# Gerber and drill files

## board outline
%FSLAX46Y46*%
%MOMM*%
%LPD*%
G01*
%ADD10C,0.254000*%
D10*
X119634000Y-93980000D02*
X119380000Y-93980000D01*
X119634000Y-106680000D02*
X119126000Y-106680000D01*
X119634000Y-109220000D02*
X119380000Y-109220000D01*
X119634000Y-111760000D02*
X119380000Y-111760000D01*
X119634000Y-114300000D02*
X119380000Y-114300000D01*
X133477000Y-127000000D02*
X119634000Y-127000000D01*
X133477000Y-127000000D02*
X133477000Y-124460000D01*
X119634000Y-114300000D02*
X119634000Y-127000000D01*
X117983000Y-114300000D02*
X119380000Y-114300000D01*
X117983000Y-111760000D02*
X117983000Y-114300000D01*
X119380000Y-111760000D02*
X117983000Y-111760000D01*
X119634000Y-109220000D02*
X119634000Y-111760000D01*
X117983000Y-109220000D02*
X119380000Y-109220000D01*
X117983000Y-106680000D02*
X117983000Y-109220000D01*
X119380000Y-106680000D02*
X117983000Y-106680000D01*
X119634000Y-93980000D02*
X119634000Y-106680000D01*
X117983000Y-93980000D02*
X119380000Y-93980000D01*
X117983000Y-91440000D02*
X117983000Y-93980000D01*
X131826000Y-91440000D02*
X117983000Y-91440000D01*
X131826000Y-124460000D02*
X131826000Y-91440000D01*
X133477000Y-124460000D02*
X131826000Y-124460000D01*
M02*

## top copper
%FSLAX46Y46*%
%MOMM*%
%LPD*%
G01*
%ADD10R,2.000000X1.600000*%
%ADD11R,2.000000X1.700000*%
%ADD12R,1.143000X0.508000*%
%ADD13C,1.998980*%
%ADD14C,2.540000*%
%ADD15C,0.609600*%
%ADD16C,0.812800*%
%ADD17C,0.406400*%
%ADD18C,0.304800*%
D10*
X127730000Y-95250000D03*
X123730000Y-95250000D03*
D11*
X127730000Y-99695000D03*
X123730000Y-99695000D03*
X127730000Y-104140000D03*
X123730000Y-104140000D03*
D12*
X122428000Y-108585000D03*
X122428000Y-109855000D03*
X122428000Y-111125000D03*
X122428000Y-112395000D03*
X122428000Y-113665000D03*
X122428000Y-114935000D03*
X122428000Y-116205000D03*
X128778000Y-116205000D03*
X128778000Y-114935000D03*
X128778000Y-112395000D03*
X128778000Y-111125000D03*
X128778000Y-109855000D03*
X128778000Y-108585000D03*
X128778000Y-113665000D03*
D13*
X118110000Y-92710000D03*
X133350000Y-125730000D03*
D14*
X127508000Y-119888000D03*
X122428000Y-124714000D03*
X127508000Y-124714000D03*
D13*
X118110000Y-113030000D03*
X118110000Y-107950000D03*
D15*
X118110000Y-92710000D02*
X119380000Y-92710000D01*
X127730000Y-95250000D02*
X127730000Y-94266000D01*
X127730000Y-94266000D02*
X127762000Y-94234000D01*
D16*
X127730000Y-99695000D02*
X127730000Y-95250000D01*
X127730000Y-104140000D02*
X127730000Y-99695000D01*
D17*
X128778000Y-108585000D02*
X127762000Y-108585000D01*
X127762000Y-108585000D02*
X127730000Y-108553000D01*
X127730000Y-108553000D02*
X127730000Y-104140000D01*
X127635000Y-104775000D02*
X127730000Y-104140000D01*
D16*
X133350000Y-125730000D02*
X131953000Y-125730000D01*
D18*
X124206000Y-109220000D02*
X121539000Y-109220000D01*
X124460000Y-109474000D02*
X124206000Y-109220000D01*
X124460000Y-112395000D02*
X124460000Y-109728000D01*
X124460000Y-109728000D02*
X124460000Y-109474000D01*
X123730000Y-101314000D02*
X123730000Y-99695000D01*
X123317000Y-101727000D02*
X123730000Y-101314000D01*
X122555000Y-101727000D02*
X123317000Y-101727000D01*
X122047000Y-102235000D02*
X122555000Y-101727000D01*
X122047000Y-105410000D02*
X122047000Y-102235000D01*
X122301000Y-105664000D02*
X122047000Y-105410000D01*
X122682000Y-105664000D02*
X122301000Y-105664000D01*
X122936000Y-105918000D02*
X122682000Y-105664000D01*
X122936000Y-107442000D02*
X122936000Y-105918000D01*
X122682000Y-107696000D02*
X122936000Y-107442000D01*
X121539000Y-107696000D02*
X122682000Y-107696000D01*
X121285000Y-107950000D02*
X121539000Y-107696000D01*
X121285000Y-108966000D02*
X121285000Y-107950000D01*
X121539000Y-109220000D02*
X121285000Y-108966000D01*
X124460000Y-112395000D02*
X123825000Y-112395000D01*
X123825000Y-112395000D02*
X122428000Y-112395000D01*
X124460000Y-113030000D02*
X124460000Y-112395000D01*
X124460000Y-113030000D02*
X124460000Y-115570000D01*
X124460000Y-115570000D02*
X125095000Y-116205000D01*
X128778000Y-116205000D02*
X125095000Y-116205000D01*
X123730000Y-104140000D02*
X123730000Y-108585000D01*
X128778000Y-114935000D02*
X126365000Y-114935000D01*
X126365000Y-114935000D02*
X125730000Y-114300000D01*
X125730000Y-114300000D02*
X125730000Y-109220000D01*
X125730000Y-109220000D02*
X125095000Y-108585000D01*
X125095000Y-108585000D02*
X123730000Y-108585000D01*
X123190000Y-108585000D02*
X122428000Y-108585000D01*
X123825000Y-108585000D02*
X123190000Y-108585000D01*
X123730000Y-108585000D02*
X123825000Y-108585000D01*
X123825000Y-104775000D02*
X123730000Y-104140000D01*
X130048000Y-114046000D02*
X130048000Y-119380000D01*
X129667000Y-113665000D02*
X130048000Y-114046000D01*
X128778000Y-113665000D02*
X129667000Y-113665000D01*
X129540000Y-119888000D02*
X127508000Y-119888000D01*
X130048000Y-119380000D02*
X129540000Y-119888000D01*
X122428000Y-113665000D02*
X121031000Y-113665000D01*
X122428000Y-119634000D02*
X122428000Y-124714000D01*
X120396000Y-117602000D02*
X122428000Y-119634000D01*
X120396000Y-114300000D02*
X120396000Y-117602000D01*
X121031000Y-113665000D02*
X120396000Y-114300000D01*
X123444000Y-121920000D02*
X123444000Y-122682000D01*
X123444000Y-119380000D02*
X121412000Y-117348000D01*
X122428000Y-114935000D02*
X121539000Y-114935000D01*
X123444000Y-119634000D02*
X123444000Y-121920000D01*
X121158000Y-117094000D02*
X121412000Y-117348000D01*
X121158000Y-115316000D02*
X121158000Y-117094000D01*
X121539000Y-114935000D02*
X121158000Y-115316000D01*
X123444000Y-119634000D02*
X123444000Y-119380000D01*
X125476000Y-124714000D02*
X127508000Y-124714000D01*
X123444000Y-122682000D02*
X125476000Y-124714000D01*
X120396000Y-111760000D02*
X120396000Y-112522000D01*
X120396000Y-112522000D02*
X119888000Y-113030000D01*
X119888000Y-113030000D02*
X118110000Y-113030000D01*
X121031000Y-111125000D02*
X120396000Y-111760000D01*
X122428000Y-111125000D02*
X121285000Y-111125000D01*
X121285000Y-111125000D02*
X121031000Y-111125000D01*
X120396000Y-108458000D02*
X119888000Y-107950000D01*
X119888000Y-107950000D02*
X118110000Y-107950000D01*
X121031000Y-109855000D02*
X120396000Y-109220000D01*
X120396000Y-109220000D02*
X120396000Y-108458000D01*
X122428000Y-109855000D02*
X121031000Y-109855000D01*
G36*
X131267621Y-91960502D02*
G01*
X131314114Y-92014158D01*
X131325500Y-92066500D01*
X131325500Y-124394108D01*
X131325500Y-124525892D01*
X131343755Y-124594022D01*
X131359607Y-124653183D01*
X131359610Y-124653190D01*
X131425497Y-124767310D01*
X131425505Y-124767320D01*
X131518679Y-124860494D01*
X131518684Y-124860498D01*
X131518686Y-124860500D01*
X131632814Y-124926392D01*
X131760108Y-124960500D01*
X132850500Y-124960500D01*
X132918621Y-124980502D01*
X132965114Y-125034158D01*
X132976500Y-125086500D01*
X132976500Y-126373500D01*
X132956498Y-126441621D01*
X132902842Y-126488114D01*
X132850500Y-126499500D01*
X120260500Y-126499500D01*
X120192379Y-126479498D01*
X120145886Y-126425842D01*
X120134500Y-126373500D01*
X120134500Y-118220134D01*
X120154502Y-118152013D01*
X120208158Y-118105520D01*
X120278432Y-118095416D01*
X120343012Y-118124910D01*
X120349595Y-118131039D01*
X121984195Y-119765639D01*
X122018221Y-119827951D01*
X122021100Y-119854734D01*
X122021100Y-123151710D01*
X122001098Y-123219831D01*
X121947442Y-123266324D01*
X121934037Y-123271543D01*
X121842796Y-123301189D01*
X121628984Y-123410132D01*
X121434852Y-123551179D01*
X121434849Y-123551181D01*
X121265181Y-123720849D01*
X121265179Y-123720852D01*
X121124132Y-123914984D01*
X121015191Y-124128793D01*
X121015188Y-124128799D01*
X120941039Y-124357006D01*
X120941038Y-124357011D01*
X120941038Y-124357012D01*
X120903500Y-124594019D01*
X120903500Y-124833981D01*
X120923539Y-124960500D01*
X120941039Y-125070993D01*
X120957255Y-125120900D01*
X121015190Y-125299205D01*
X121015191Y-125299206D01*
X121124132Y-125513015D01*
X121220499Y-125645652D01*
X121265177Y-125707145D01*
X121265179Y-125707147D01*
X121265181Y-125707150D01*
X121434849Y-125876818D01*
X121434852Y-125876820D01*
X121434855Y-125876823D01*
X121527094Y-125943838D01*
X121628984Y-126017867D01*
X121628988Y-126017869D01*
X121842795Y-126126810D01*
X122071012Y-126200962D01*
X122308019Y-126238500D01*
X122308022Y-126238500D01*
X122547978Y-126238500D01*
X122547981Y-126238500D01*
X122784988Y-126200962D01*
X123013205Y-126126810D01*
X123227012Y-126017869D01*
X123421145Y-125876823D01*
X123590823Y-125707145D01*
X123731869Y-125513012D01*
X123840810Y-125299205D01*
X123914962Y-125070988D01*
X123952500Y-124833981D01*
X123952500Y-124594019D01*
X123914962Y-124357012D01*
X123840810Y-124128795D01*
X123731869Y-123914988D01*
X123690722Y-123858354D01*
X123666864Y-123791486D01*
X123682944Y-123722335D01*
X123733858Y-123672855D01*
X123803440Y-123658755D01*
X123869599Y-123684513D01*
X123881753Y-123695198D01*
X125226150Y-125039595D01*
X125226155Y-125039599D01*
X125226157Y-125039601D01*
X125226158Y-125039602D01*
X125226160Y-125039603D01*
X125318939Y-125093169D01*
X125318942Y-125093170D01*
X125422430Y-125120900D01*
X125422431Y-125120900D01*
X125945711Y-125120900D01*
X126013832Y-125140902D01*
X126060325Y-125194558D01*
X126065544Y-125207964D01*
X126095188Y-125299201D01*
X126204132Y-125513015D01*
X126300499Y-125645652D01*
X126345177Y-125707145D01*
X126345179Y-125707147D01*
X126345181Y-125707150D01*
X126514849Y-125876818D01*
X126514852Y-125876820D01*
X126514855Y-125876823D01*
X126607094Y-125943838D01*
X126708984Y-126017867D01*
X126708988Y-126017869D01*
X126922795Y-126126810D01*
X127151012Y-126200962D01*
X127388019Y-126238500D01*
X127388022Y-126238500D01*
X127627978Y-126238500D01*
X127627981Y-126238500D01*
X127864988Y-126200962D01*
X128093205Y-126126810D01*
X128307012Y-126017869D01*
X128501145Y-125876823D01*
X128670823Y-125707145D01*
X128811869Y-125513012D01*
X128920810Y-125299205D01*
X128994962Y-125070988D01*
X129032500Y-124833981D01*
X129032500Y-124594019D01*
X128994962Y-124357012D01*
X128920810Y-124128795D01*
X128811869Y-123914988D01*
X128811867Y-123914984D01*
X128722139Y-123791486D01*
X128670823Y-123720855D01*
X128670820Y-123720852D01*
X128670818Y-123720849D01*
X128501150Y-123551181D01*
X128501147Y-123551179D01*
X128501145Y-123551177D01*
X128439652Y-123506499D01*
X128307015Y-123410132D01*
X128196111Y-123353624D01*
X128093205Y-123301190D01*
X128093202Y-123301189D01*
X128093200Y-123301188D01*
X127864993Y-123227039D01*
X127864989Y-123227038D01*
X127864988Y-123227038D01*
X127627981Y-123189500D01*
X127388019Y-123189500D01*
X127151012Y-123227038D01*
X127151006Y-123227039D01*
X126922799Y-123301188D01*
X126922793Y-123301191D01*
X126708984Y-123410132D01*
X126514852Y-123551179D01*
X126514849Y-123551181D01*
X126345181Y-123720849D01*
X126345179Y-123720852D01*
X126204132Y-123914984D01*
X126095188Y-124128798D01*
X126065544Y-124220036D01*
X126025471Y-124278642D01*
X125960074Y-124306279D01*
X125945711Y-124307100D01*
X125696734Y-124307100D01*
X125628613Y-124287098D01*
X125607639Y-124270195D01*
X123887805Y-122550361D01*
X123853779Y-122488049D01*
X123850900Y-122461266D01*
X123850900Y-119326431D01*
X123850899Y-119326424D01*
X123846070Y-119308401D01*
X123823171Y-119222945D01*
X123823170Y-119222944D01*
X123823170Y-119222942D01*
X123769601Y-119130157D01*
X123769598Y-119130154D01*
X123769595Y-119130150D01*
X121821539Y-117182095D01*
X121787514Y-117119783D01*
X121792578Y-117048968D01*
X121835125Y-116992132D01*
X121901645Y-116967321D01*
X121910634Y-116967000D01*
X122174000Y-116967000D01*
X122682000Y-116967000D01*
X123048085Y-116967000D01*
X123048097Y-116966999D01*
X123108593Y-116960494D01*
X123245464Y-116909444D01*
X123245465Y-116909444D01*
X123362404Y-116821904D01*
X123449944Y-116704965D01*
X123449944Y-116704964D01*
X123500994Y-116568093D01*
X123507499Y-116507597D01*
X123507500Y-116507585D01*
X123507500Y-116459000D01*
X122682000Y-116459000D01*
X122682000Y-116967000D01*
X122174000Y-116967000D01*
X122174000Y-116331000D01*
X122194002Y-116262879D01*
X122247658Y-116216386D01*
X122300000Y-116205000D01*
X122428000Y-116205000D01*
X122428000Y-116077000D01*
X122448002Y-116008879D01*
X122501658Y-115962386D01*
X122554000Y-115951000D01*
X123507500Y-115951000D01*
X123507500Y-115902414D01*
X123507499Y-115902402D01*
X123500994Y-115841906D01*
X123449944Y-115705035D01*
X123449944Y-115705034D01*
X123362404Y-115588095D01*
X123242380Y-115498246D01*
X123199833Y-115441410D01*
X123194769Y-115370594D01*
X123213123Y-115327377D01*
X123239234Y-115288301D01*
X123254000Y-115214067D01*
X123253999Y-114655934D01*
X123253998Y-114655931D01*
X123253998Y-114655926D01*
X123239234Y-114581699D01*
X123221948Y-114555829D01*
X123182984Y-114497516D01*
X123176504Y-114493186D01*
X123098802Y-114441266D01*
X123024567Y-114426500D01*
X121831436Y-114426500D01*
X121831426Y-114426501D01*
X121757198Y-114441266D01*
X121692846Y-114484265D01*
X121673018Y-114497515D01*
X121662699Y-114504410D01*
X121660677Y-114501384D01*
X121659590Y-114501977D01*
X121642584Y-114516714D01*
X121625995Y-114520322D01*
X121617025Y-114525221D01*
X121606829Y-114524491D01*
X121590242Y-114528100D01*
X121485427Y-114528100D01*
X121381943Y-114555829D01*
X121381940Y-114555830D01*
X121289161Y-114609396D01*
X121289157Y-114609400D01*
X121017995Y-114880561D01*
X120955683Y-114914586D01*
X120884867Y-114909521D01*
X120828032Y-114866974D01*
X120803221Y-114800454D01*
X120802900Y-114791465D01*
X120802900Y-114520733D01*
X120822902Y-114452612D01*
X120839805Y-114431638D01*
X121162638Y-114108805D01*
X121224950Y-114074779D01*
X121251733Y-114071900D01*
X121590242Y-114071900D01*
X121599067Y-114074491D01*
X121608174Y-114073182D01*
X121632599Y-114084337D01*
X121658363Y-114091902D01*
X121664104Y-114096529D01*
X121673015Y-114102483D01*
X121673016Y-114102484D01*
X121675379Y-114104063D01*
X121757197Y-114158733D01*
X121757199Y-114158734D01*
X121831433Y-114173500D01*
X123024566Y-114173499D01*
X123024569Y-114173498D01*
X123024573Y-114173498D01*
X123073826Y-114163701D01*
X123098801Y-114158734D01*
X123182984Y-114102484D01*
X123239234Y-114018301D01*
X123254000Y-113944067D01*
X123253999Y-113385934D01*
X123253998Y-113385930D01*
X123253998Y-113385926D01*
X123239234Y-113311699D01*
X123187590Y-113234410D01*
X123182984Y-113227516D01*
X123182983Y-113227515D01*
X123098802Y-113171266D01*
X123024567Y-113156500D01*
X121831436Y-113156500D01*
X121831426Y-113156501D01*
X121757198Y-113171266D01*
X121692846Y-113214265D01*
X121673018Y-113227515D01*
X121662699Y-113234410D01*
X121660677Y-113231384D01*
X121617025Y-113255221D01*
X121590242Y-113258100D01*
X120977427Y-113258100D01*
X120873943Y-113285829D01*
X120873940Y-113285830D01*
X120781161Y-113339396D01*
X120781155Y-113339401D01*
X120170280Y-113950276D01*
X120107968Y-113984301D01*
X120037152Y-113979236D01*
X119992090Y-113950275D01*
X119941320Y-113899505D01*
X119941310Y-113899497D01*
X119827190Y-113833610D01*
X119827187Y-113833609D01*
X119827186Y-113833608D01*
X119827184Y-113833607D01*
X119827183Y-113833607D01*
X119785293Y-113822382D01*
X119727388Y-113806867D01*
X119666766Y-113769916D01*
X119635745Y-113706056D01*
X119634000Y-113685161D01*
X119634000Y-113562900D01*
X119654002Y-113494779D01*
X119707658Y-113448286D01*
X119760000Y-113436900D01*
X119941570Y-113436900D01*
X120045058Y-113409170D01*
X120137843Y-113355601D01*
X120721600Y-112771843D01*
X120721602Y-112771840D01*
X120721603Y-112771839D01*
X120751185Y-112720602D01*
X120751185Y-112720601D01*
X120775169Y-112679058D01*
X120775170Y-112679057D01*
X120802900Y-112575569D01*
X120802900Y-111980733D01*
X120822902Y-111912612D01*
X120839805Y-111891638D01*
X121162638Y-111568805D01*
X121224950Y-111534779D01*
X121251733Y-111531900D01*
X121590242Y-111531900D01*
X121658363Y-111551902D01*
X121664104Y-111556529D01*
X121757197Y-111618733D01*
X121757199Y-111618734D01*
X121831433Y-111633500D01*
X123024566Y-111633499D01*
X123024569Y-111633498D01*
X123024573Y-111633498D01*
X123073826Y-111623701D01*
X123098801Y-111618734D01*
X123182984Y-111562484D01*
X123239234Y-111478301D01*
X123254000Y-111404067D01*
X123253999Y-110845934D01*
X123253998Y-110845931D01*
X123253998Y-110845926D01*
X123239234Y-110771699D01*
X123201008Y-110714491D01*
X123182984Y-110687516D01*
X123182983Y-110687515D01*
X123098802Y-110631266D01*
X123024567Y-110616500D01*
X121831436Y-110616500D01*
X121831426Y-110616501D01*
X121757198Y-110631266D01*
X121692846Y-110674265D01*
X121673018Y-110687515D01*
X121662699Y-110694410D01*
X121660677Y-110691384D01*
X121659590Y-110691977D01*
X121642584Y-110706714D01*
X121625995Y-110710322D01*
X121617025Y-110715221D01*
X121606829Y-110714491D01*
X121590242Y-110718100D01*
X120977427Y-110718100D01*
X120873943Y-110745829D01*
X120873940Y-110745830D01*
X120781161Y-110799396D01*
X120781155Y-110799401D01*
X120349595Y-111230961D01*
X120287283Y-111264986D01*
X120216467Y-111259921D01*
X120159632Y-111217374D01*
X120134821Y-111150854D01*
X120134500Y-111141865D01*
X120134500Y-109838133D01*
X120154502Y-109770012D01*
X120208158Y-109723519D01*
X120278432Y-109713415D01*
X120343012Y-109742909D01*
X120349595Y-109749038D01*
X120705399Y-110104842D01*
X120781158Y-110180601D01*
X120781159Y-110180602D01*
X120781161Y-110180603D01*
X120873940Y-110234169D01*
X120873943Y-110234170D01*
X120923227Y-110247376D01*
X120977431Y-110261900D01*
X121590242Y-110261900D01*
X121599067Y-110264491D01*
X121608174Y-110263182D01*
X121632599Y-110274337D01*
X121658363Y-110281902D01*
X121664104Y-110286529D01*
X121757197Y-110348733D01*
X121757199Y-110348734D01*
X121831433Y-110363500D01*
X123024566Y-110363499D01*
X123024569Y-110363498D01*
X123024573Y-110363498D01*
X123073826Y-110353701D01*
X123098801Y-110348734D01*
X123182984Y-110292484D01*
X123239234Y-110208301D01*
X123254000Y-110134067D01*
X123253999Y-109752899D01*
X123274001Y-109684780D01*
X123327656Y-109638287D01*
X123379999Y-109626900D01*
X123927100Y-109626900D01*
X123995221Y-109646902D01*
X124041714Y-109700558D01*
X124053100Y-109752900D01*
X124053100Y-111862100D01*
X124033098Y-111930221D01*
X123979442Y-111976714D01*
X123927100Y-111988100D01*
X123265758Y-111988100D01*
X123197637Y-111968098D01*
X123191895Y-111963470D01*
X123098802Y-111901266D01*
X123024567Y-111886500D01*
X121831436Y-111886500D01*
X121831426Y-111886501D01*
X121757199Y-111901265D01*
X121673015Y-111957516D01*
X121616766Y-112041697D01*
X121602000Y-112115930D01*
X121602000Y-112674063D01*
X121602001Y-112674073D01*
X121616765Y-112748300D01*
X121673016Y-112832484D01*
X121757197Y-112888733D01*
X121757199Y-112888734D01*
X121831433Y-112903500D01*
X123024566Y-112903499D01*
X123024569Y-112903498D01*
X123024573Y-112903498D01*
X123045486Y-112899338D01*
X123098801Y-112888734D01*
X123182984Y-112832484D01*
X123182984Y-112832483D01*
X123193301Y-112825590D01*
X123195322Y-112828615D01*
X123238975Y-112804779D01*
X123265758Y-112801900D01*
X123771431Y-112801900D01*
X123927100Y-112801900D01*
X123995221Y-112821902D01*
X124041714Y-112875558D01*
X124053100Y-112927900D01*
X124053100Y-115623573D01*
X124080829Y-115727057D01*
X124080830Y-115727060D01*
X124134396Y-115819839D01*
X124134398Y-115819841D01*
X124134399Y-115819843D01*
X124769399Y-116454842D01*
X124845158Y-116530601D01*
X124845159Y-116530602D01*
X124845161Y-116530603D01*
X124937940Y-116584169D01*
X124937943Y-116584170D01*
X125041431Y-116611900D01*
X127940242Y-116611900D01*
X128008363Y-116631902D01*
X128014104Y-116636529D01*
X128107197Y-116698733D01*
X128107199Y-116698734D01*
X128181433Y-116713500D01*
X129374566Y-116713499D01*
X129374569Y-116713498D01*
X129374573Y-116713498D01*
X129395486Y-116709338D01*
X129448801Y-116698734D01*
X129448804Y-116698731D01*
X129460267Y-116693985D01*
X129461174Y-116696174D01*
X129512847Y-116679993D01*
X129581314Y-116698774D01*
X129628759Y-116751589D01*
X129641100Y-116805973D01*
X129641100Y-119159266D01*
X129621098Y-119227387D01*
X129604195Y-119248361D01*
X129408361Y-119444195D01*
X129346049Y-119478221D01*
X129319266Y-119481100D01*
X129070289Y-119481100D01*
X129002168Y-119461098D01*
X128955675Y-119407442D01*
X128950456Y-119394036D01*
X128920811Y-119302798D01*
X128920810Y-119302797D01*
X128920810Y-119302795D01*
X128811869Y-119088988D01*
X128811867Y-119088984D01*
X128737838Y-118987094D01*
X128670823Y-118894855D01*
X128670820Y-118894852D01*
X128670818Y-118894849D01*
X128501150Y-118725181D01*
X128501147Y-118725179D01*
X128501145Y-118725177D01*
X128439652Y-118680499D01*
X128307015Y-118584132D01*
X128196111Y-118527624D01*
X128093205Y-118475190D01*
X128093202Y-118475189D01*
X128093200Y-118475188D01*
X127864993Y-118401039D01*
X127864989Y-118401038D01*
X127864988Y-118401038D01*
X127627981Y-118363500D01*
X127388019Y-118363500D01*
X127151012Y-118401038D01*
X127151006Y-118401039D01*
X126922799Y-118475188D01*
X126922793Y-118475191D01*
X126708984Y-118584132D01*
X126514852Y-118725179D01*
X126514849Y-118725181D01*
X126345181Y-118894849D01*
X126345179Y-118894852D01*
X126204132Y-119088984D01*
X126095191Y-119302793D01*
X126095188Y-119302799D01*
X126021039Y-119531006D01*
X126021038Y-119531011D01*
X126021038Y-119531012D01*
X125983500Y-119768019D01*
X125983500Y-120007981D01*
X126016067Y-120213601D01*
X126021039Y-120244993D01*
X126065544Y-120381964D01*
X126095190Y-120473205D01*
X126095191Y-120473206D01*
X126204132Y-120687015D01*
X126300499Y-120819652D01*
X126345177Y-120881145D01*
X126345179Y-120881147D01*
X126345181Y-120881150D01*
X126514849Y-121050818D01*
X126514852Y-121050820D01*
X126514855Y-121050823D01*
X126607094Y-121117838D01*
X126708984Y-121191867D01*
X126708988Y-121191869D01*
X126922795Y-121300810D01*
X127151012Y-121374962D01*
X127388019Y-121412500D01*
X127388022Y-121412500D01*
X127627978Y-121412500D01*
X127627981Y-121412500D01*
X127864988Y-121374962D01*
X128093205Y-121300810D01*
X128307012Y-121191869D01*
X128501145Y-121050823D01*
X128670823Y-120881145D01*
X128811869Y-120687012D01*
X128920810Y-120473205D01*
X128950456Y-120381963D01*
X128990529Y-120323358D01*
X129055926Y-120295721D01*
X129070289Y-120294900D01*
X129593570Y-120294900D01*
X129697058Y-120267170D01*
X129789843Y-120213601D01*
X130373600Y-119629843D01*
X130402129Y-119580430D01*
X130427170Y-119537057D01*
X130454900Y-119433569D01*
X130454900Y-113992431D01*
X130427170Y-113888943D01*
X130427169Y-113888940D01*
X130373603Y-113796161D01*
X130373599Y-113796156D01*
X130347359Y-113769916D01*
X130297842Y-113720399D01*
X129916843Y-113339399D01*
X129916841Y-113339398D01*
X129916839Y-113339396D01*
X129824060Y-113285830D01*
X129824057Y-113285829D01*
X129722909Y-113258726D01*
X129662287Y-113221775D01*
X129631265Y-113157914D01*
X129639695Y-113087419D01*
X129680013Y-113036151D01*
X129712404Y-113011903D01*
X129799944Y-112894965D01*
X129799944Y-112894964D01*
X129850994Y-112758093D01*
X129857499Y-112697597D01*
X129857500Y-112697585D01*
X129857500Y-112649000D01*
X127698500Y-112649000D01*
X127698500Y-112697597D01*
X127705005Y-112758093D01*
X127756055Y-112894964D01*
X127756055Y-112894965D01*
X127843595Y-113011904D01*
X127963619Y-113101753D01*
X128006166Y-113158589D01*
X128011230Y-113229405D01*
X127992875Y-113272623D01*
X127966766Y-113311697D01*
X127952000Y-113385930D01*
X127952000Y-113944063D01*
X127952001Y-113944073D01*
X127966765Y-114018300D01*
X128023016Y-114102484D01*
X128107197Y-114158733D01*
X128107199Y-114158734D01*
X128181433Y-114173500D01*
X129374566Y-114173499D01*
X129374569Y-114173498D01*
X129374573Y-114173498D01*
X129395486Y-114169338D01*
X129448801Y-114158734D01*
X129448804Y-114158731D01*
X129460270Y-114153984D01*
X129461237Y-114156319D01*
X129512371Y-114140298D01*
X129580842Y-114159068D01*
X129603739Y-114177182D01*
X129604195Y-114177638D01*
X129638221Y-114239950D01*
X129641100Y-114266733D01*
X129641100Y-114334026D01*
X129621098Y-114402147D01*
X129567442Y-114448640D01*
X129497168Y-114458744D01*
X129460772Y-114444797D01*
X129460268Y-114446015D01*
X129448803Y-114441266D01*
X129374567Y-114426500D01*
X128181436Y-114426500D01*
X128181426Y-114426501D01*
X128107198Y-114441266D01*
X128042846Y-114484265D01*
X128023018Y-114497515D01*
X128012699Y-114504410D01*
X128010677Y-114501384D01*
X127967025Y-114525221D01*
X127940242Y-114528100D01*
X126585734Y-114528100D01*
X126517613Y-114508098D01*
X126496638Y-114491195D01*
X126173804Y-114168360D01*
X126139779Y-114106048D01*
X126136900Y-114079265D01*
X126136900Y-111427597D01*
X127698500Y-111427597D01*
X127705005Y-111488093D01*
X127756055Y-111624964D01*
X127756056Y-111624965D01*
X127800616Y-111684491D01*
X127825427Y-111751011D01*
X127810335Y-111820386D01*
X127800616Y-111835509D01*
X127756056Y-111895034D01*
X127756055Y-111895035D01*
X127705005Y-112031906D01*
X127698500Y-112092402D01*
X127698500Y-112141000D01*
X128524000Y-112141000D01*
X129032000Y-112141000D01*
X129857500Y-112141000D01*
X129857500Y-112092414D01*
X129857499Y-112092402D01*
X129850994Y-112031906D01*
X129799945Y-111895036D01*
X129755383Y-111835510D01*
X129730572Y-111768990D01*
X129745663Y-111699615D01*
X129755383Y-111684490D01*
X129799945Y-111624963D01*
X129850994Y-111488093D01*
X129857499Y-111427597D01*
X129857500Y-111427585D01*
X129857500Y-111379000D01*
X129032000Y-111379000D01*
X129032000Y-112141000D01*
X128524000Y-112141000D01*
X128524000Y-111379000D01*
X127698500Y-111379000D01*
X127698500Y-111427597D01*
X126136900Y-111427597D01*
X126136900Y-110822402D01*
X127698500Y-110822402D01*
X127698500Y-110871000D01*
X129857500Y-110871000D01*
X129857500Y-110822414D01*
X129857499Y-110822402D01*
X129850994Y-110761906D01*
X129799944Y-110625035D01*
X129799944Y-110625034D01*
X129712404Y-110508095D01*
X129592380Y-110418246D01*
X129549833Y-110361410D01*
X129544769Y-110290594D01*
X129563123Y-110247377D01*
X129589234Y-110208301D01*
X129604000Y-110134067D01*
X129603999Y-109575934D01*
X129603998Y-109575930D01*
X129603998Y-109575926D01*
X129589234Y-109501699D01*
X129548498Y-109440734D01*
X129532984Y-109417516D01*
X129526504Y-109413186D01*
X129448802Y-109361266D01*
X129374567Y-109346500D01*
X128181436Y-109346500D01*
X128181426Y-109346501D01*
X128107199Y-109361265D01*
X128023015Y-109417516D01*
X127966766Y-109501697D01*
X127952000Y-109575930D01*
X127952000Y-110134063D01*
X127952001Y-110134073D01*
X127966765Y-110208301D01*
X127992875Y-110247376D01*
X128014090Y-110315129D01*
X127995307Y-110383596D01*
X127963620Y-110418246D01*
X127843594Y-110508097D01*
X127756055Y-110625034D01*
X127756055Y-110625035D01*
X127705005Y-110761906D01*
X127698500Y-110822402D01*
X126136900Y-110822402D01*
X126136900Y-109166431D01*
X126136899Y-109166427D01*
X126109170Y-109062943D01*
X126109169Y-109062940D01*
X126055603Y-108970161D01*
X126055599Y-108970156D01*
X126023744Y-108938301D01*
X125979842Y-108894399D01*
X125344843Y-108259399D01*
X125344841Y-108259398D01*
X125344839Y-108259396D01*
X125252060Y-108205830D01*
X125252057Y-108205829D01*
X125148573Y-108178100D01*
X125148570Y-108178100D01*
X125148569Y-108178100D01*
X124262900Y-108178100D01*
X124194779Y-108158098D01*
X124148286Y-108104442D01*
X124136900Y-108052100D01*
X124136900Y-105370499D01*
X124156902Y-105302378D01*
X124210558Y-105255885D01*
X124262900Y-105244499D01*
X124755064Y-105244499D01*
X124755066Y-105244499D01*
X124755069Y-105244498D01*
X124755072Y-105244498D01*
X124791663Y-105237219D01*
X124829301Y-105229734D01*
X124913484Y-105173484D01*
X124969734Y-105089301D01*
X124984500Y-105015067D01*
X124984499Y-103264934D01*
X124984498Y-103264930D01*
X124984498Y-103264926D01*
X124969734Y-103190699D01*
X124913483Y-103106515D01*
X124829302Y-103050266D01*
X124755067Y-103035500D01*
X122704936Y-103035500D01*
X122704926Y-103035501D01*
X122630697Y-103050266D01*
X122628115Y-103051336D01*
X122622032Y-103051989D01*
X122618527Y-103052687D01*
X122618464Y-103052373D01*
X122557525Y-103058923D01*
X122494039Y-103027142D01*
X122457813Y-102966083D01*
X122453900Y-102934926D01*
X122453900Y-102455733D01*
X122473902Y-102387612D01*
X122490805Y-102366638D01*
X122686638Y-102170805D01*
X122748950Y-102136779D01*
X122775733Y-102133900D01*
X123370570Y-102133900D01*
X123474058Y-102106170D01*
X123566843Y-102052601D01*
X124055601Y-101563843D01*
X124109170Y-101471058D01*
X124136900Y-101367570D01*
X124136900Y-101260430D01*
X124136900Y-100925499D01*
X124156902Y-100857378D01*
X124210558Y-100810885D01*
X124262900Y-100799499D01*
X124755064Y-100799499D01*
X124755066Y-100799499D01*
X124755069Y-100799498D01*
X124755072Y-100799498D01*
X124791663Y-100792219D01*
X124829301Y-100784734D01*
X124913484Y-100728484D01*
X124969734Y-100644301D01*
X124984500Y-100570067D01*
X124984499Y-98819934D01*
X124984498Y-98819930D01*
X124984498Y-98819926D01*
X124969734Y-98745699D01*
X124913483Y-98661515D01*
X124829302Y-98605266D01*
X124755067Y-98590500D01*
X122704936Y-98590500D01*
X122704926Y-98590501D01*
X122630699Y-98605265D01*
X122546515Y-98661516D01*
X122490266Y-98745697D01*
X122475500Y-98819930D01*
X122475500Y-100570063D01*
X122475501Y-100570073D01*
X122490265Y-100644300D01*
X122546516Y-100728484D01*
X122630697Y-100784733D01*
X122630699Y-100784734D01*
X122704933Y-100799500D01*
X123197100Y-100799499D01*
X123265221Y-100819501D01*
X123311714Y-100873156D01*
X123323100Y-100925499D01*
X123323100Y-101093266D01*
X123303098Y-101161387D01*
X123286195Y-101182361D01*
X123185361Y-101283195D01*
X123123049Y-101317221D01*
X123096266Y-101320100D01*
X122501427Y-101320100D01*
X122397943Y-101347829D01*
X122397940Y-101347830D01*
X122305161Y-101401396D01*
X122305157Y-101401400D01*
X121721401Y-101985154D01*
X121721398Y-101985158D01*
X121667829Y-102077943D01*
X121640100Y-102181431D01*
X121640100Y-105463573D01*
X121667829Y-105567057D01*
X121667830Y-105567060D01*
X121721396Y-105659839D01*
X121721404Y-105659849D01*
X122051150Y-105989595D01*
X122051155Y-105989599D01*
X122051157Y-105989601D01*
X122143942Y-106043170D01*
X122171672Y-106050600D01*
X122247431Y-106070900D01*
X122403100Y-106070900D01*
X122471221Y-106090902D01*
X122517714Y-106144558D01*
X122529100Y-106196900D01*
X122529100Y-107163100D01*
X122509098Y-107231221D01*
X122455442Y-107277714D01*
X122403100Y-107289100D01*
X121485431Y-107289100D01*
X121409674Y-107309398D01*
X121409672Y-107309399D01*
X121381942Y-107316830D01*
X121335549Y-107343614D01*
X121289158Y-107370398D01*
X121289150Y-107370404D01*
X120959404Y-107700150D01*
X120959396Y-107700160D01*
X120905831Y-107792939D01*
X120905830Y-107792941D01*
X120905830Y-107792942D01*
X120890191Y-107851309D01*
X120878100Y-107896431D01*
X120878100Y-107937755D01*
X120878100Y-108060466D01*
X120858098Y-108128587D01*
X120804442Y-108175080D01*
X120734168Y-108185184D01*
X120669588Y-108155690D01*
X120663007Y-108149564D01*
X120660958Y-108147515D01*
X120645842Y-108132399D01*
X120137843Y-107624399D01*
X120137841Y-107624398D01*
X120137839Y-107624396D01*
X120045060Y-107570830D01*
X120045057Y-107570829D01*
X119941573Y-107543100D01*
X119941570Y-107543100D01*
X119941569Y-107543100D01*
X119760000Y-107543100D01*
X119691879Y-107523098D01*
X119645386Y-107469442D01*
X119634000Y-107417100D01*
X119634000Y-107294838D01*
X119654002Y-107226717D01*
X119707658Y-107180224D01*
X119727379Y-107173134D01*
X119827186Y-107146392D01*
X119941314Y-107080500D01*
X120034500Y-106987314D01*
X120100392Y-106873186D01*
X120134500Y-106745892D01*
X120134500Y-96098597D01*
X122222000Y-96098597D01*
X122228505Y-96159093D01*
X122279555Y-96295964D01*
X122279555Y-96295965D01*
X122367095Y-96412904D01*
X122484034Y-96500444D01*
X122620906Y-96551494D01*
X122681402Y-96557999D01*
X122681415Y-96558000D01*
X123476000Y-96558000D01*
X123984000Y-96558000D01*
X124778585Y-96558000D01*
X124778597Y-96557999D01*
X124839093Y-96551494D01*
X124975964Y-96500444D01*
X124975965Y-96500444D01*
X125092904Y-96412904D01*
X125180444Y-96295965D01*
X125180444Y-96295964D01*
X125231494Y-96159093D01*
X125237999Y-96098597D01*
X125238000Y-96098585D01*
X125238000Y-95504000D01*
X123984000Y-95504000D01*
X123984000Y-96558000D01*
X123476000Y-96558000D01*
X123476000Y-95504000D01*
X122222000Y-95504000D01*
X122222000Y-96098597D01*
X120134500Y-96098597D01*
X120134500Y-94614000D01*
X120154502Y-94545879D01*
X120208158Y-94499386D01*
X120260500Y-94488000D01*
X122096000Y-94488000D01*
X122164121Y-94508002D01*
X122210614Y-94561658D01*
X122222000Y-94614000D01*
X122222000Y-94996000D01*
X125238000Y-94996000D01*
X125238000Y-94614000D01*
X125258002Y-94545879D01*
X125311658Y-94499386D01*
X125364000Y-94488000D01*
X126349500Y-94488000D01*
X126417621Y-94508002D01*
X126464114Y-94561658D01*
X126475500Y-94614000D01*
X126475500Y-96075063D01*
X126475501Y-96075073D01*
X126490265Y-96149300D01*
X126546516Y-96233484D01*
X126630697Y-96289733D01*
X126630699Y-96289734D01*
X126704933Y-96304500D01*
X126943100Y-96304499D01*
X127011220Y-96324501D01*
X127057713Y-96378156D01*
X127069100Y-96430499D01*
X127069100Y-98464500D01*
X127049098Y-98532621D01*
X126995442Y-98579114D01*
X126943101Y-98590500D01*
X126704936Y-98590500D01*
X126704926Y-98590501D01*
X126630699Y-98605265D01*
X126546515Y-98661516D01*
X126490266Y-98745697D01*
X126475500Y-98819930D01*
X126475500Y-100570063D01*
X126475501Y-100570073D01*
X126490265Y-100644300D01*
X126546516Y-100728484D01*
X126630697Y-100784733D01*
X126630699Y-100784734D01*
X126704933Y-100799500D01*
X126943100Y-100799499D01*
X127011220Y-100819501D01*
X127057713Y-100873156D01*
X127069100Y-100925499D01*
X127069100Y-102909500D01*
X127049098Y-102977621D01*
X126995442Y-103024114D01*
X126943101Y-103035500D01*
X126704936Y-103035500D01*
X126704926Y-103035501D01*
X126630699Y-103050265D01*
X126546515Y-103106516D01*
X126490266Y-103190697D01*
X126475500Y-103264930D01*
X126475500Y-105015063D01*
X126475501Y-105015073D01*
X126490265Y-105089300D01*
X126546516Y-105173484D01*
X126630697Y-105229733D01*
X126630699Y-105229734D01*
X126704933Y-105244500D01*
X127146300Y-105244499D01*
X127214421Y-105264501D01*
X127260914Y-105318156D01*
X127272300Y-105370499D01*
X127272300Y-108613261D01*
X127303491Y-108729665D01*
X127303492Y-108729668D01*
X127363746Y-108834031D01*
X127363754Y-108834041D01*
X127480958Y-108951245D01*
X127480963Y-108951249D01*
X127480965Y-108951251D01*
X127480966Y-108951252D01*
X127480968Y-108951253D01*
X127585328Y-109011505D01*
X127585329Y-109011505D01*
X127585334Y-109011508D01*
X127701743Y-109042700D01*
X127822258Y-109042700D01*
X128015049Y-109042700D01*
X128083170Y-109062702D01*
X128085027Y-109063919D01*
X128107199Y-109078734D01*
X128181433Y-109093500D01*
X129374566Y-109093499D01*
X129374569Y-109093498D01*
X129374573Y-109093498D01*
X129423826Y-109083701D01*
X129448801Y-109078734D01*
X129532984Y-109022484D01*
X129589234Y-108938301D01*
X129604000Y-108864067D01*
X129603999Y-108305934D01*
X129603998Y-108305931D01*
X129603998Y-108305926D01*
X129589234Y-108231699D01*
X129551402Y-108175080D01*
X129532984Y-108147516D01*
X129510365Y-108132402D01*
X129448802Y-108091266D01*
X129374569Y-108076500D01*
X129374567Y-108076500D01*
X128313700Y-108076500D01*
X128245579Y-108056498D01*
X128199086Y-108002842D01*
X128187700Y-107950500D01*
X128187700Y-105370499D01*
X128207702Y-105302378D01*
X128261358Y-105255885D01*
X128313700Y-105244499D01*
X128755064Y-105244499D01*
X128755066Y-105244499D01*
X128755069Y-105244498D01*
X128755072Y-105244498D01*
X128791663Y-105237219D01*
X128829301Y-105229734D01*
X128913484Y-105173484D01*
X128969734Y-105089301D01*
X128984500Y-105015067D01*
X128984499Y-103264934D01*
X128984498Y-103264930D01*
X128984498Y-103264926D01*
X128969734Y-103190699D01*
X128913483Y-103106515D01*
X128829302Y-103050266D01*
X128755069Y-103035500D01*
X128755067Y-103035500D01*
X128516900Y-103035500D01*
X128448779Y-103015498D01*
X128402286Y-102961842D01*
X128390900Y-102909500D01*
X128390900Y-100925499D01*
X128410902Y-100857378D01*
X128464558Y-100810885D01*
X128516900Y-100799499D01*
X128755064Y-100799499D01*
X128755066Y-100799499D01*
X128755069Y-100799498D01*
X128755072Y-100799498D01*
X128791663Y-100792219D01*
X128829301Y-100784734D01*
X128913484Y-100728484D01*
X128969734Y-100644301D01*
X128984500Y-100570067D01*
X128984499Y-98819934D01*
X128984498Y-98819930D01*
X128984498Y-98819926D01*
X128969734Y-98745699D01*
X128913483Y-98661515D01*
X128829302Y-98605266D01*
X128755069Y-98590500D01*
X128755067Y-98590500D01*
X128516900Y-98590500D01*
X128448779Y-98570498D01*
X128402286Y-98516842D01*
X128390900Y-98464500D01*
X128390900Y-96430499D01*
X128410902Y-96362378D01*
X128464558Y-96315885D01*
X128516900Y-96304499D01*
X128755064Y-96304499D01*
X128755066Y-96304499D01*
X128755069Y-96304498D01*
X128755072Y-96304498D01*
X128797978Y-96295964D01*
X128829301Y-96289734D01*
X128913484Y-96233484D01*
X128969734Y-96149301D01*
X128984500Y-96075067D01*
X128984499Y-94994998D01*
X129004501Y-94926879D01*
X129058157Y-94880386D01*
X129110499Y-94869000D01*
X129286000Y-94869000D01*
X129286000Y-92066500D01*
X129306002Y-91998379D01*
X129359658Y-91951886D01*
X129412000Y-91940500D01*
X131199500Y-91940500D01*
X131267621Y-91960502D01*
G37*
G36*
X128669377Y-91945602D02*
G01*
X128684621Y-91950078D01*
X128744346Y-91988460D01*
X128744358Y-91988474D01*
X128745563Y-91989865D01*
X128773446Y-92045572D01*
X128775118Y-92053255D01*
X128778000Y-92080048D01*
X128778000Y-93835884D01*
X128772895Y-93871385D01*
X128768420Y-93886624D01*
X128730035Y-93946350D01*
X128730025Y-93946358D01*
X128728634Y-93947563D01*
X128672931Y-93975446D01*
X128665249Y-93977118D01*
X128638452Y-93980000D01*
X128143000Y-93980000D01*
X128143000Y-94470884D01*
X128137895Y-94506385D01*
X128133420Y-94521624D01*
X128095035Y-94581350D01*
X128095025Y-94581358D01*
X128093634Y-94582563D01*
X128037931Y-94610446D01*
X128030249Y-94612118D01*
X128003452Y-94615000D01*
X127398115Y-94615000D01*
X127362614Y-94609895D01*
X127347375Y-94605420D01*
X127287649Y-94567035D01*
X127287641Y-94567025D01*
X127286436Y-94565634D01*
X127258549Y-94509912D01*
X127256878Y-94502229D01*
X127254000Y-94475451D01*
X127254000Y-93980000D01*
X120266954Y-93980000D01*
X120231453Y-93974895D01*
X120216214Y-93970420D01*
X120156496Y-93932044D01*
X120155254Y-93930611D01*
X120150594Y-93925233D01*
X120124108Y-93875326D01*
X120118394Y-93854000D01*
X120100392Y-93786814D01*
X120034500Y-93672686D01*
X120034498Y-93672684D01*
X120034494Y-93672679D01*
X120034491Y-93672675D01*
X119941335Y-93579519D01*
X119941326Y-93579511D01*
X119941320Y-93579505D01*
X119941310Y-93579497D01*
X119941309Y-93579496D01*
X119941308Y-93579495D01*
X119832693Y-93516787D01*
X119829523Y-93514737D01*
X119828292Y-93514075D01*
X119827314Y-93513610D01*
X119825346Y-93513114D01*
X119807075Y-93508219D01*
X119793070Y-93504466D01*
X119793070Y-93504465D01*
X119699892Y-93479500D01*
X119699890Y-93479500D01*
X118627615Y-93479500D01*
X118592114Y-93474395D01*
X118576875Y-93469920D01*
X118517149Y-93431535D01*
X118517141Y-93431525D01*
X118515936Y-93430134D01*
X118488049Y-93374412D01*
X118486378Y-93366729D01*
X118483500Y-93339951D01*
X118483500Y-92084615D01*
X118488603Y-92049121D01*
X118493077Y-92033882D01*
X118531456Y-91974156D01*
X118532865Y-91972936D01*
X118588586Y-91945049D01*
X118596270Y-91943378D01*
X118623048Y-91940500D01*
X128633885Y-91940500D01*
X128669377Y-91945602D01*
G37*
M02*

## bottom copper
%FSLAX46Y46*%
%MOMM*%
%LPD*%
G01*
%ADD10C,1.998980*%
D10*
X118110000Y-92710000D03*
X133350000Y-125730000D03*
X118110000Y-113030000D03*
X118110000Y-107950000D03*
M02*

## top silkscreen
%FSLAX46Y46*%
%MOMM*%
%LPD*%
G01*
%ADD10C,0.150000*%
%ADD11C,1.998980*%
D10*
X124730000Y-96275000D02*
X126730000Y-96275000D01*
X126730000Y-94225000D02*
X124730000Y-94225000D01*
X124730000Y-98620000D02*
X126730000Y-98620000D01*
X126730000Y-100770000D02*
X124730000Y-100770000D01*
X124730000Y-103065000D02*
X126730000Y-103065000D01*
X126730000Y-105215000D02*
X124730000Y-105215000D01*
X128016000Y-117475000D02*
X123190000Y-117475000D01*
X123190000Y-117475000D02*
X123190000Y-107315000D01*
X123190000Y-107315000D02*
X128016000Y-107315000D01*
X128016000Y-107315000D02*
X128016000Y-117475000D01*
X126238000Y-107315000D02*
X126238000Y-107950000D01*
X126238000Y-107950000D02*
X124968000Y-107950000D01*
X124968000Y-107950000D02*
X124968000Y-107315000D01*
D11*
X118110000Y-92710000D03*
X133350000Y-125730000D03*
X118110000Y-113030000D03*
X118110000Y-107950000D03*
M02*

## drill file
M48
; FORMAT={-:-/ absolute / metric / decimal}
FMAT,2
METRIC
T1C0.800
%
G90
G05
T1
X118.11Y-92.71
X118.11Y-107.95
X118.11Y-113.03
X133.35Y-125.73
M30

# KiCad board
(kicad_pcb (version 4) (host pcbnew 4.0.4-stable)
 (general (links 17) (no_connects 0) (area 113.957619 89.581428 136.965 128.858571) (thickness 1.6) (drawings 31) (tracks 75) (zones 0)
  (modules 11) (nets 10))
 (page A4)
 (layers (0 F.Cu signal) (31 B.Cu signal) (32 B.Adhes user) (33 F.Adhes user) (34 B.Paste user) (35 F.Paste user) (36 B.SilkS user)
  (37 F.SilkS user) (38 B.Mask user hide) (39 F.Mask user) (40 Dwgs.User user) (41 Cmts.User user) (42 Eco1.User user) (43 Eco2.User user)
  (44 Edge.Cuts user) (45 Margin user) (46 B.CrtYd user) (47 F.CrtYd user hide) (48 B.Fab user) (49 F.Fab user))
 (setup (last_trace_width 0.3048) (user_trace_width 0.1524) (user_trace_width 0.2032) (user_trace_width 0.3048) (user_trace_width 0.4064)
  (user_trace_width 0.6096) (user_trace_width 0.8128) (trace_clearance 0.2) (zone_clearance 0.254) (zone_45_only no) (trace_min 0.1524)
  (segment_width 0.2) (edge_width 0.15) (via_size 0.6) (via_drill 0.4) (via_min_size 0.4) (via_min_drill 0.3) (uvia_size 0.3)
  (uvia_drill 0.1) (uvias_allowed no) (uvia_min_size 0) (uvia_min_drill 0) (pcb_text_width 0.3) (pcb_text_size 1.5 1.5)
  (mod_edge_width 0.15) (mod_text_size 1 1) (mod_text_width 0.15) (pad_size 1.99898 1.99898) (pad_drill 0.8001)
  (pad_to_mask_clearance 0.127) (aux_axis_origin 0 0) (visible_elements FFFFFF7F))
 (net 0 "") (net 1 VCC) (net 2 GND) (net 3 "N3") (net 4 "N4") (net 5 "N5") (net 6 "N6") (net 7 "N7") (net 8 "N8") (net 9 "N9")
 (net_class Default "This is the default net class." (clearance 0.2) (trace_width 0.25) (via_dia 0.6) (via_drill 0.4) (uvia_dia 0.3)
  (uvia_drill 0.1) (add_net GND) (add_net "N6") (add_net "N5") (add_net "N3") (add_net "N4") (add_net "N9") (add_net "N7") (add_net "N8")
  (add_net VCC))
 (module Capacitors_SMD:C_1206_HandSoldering (layer F.Cu) (at 125.73 95.25 180)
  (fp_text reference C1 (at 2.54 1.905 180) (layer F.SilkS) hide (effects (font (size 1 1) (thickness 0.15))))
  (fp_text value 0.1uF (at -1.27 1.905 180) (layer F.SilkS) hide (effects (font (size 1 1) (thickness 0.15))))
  (fp_line (start 1 -1.025) (end -1 -1.025) (layer F.SilkS) (width 0.15))
  (fp_line (start -1 1.025) (end 1 1.025) (layer F.SilkS) (width 0.15))
  (pad 1 smd rect (at -2 0 180) (size 2 1.6) (layers F.Cu F.Paste F.Mask) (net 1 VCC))
  (pad 2 smd rect (at 2 0 180) (size 2 1.6) (layers F.Cu F.Paste F.Mask) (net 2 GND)))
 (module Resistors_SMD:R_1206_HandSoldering (layer F.Cu) (at 125.73 99.695 180)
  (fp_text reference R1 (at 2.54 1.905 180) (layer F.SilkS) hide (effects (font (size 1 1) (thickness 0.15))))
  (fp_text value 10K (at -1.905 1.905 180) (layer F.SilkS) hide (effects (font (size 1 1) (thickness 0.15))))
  (fp_line (start 1 1.075) (end -1 1.075) (layer F.SilkS) (width 0.15))
  (fp_line (start -1 -1.075) (end 1 -1.075) (layer F.SilkS) (width 0.15))
  (pad 1 smd rect (at -2 0 180) (size 2 1.7) (layers F.Cu F.Paste F.Mask) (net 1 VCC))
  (pad 2 smd rect (at 2 0 180) (size 2 1.7) (layers F.Cu F.Paste F.Mask) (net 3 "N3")))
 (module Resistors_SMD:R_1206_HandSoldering (layer F.Cu) (at 125.73 104.14 180)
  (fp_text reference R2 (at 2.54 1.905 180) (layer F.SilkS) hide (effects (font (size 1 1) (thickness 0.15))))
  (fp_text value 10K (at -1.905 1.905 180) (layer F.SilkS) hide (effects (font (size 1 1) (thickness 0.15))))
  (fp_line (start 1 1.075) (end -1 1.075) (layer F.SilkS) (width 0.15))
  (fp_line (start -1 -1.075) (end 1 -1.075) (layer F.SilkS) (width 0.15))
  (pad 1 smd rect (at -2 0 180) (size 2 1.7) (layers F.Cu F.Paste F.Mask) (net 1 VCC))
  (pad 2 smd rect (at 2 0 180) (size 2 1.7) (layers F.Cu F.Paste F.Mask) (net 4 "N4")))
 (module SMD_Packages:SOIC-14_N (layer F.Cu) (at 125.73 112.395 270)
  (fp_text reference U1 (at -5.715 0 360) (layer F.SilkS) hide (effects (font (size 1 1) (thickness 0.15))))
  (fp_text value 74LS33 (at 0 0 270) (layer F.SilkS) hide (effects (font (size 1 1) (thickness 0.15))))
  (fp_line (start 5.08 -2.286) (end 5.08 2.54) (layer F.SilkS) (width 0.15))
  (fp_line (start 5.08 2.54) (end -5.08 2.54) (layer F.SilkS) (width 0.15))
  (fp_line (start -5.08 2.54) (end -5.08 -2.286) (layer F.SilkS) (width 0.15))
  (fp_line (start -5.08 -2.286) (end 5.08 -2.286) (layer F.SilkS) (width 0.15))
  (fp_line (start -5.08 -0.508) (end -4.445 -0.508) (layer F.SilkS) (width 0.15))
  (fp_line (start -4.445 -0.508) (end -4.445 0.762) (layer F.SilkS) (width 0.15))
  (fp_line (start -4.445 0.762) (end -5.08 0.762) (layer F.SilkS) (width 0.15))
  (pad 1 smd rect (at -3.81 3.302 270) (size 0.508 1.143) (layers F.Cu F.Paste F.Mask) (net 4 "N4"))
  (pad 2 smd rect (at -2.54 3.302 270) (size 0.508 1.143) (layers F.Cu F.Paste F.Mask) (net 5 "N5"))
  (pad 3 smd rect (at -1.27 3.302 270) (size 0.508 1.143) (layers F.Cu F.Paste F.Mask) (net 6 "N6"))
  (pad 4 smd rect (at 0 3.302 270) (size 0.508 1.143) (layers F.Cu F.Paste F.Mask) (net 3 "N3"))
  (pad 5 smd rect (at 1.27 3.302 270) (size 0.508 1.143) (layers F.Cu F.Paste F.Mask) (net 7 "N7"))
  (pad 6 smd rect (at 2.54 3.302 270) (size 0.508 1.143) (layers F.Cu F.Paste F.Mask) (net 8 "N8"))
  (pad 7 smd rect (at 3.81 3.302 270) (size 0.508 1.143) (layers F.Cu F.Paste F.Mask) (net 2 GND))
  (pad 8 smd rect (at 3.81 -3.048 270) (size 0.508 1.143) (layers F.Cu F.Paste F.Mask) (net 3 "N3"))
  (pad 9 smd rect (at 2.54 -3.048 270) (size 0.508 1.143) (layers F.Cu F.Paste F.Mask) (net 4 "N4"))
  (pad 11 smd rect (at 0 -3.048 270) (size 0.508 1.143) (layers F.Cu F.Paste F.Mask) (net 2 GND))
  (pad 12 smd rect (at -1.27 -3.048 270) (size 0.508 1.143) (layers F.Cu F.Paste F.Mask) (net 2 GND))
  (pad 13 smd rect (at -2.54 -3.048 270) (size 0.508 1.143) (layers F.Cu F.Paste F.Mask))
  (pad 14 smd rect (at -3.81 -3.048 270) (size 0.508 1.143) (layers F.Cu F.Paste F.Mask) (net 1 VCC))
  (pad 10 smd rect (at 1.27 -3.048 270) (size 0.508 1.143) (layers F.Cu F.Paste F.Mask) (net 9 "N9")))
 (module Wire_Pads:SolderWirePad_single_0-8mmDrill (layer F.Cu) (at 118.11 92.71 90)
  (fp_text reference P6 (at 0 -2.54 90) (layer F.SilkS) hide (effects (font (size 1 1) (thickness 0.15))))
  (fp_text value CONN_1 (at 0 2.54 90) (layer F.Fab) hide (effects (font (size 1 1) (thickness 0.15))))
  (pad 1 thru_hole circle (at 0 0 90) (size 1.99898 1.99898) (drill 0.8001) (layers *.Cu *.Mask F.SilkS) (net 1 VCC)))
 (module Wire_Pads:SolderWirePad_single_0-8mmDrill (layer F.Cu) (at 133.35 125.73 270)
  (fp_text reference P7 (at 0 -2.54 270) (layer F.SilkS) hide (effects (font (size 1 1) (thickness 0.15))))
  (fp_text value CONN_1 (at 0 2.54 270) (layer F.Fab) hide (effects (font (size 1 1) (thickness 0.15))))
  (pad 1 thru_hole circle (at 0 0 270) (size 1.99898 1.99898) (drill 0.8001) (layers *.Cu *.Mask F.SilkS) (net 2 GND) (zone_connect 2)))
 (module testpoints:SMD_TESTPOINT (layer F.Cu) (at 127.508 119.888)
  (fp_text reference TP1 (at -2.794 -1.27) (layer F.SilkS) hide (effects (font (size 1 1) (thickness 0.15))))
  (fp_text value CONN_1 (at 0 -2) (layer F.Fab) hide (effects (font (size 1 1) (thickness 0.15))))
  (pad 1 smd circle (at 0 0) (size 2.54 2.54) (layers F.Cu F.Paste F.Mask) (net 9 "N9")))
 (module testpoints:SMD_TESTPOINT (layer F.Cu) (at 122.428 124.714)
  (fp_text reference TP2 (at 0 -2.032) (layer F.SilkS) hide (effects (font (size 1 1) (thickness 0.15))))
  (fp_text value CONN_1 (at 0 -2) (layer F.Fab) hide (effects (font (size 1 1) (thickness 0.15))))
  (pad 1 smd circle (at 0 0) (size 2.54 2.54) (layers F.Cu F.Paste F.Mask) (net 7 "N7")))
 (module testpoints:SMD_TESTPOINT (layer F.Cu) (at 127.508 124.714)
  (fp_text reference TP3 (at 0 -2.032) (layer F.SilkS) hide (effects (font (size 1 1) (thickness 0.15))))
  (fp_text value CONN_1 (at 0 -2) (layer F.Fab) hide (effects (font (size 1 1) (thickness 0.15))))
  (pad 1 smd circle (at 0 0) (size 2.54 2.54) (layers F.Cu F.Paste F.Mask) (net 8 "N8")))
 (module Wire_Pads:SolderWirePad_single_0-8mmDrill (layer F.Cu) (at 118.11 113.03)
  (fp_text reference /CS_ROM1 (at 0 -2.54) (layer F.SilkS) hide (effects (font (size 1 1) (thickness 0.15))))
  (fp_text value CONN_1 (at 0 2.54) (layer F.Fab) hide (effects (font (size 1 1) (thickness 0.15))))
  (pad 1 thru_hole circle (at 0 0) (size 1.99898 1.99898) (drill 0.8001) (layers *.Cu *.Mask F.SilkS) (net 6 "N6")))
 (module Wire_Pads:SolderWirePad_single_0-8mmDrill (layer F.Cu) (at 118.11 107.95)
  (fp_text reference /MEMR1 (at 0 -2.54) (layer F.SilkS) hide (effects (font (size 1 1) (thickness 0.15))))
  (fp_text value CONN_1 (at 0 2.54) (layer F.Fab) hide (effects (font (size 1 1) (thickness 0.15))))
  (pad 1 thru_hole circle (at 0 0) (size 1.99898 1.99898) (drill 0.8001) (layers *.Cu *.Mask F.SilkS) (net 5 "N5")))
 (gr_line (start 119.634 93.98) (end 119.38 93.98) (angle 90) (layer Edge.Cuts) (width 0.254))
 (gr_line (start 119.634 106.68) (end 119.126 106.68) (angle 90) (layer Edge.Cuts) (width 0.254))
 (gr_line (start 119.634 109.22) (end 119.38 109.22) (angle 90) (layer Edge.Cuts) (width 0.254))
 (gr_line (start 119.634 111.76) (end 119.38 111.76) (angle 90) (layer Edge.Cuts) (width 0.254))
 (gr_line (start 119.634 114.3) (end 119.38 114.3) (angle 90) (layer Edge.Cuts) (width 0.254))
 (gr_line (start 133.477 127) (end 119.634 127) (angle 90) (layer Edge.Cuts) (width 0.254))
 (gr_line (start 133.477 127) (end 133.477 124.46) (angle 90) (layer Edge.Cuts) (width 0.254))
 (gr_line (start 119.634 114.3) (end 119.634 127) (angle 90) (layer Edge.Cuts) (width 0.254))
 (gr_line (start 117.983 114.3) (end 119.38 114.3) (angle 90) (layer Edge.Cuts) (width 0.254))
 (gr_line (start 117.983 111.76) (end 117.983 114.3) (angle 90) (layer Edge.Cuts) (width 0.254))
 (gr_line (start 119.38 111.76) (end 117.983 111.76) (angle 90) (layer Edge.Cuts) (width 0.254))
 (gr_line (start 119.634 109.22) (end 119.634 111.76) (angle 90) (layer Edge.Cuts) (width 0.254))
 (gr_line (start 117.983 109.22) (end 119.38 109.22) (angle 90) (layer Edge.Cuts) (width 0.254))
 (gr_line (start 117.983 106.68) (end 117.983 109.22) (angle 90) (layer Edge.Cuts) (width 0.254))
 (gr_line (start 119.38 106.68) (end 117.983 106.68) (angle 90) (layer Edge.Cuts) (width 0.254))
 (gr_line (start 119.634 93.98) (end 119.634 106.68) (angle 90) (layer Edge.Cuts) (width 0.254))
 (gr_line (start 117.983 93.98) (end 119.38 93.98) (angle 90) (layer Edge.Cuts) (width 0.254))
 (gr_line (start 117.983 91.44) (end 117.983 93.98) (angle 90) (layer Edge.Cuts) (width 0.254))
 (gr_line (start 131.826 91.44) (end 117.983 91.44) (angle 90) (layer Edge.Cuts) (width 0.254))
 (gr_line (start 131.826 124.46) (end 131.826 91.44) (angle 90) (layer Edge.Cuts) (width 0.254))
 (gr_line (start 133.477 124.46) (end 131.826 124.46) (angle 90) (layer Edge.Cuts) (width 0.254))
 (segment (start 118.11 92.71) (end 119.38 92.71) (width 0.6096) (layer F.Cu) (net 1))
 (segment (start 127.73 95.25) (end 127.73 94.266) (width 0.6096) (layer F.Cu) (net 1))
 (segment (start 127.73 94.266) (end 127.762 94.234) (width 0.6096) (layer F.Cu) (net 1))
 (segment (start 127.73 99.695) (end 127.73 95.25) (width 0.8128) (layer F.Cu) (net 1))
 (segment (start 127.73 104.14) (end 127.73 99.695) (width 0.8128) (layer F.Cu) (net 1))
 (segment (start 128.778 108.585) (end 127.762 108.585) (width 0.4064) (layer F.Cu) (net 1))
 (segment (start 127.762 108.585) (end 127.73 108.553) (width 0.4064) (layer F.Cu) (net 1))
 (segment (start 127.73 108.553) (end 127.73 104.14) (width 0.4064) (layer F.Cu) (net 1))
 (segment (start 127.635 104.775) (end 127.73 104.14) (width 0.4064) (layer F.Cu) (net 1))
 (segment (start 133.35 125.73) (end 131.953 125.73) (width 0.8128) (layer F.Cu) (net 2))
 (segment (start 124.206 109.22) (end 121.539 109.22) (width 0.3048) (layer F.Cu) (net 3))
 (segment (start 124.46 109.474) (end 124.206 109.22) (width 0.3048) (layer F.Cu) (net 3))
 (segment (start 124.46 112.395) (end 124.46 109.728) (width 0.3048) (layer F.Cu) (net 3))
 (segment (start 124.46 109.728) (end 124.46 109.474) (width 0.3048) (layer F.Cu) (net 3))
 (segment (start 123.73 101.314) (end 123.73 99.695) (width 0.3048) (layer F.Cu) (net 3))
 (segment (start 123.317 101.727) (end 123.73 101.314) (width 0.3048) (layer F.Cu) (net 3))
 (segment (start 122.555 101.727) (end 123.317 101.727) (width 0.3048) (layer F.Cu) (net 3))
 (segment (start 122.047 102.235) (end 122.555 101.727) (width 0.3048) (layer F.Cu) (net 3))
 (segment (start 122.047 105.41) (end 122.047 102.235) (width 0.3048) (layer F.Cu) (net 3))
 (segment (start 122.301 105.664) (end 122.047 105.41) (width 0.3048) (layer F.Cu) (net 3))
 (segment (start 122.682 105.664) (end 122.301 105.664) (width 0.3048) (layer F.Cu) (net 3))
 (segment (start 122.936 105.918) (end 122.682 105.664) (width 0.3048) (layer F.Cu) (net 3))
 (segment (start 122.936 107.442) (end 122.936 105.918) (width 0.3048) (layer F.Cu) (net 3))
 (segment (start 122.682 107.696) (end 122.936 107.442) (width 0.3048) (layer F.Cu) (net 3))
 (segment (start 121.539 107.696) (end 122.682 107.696) (width 0.3048) (layer F.Cu) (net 3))
 (segment (start 121.285 107.95) (end 121.539 107.696) (width 0.3048) (layer F.Cu) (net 3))
 (segment (start 121.285 108.966) (end 121.285 107.95) (width 0.3048) (layer F.Cu) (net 3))
 (segment (start 121.539 109.22) (end 121.285 108.966) (width 0.3048) (layer F.Cu) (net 3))
 (segment (start 124.46 112.395) (end 123.825 112.395) (width 0.3048) (layer F.Cu) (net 3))
 (segment (start 123.825 112.395) (end 122.428 112.395) (width 0.3048) (layer F.Cu) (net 3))
 (segment (start 124.46 113.03) (end 124.46 112.395) (width 0.3048) (layer F.Cu) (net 3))
 (segment (start 124.46 113.03) (end 124.46 115.57) (width 0.3048) (layer F.Cu) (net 3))
 (segment (start 124.46 115.57) (end 125.095 116.205) (width 0.3048) (layer F.Cu) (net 3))
 (segment (start 128.778 116.205) (end 125.095 116.205) (width 0.3048) (layer F.Cu) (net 3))
 (segment (start 123.73 104.14) (end 123.73 108.585) (width 0.3048) (layer F.Cu) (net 4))
 (segment (start 128.778 114.935) (end 126.365 114.935) (width 0.3048) (layer F.Cu) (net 4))
 (segment (start 126.365 114.935) (end 125.73 114.3) (width 0.3048) (layer F.Cu) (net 4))
 (segment (start 125.73 114.3) (end 125.73 109.22) (width 0.3048) (layer F.Cu) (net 4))
 (segment (start 125.73 109.22) (end 125.095 108.585) (width 0.3048) (layer F.Cu) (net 4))
 (segment (start 125.095 108.585) (end 123.73 108.585) (width 0.3048) (layer F.Cu) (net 4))
 (segment (start 123.19 108.585) (end 122.428 108.585) (width 0.3048) (layer F.Cu) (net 4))
 (segment (start 123.825 108.585) (end 123.19 108.585) (width 0.3048) (layer F.Cu) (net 4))
 (segment (start 123.73 108.585) (end 123.825 108.585) (width 0.3048) (layer F.Cu) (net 4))
 (segment (start 123.825 104.775) (end 123.73 104.14) (width 0.3048) (layer F.Cu) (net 4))
 (segment (start 130.048 114.046) (end 130.048 119.38) (width 0.3048) (layer F.Cu) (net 9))
 (segment (start 129.667 113.665) (end 130.048 114.046) (width 0.3048) (layer F.Cu) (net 9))
 (segment (start 128.778 113.665) (end 129.667 113.665) (width 0.3048) (layer F.Cu) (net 9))
 (segment (start 129.54 119.888) (end 127.508 119.888) (width 0.3048) (layer F.Cu) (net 9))
 (segment (start 130.048 119.38) (end 129.54 119.888) (width 0.3048) (layer F.Cu) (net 9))
 (segment (start 122.428 113.665) (end 121.031 113.665) (width 0.3048) (layer F.Cu) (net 7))
 (segment (start 122.428 119.634) (end 122.428 124.714) (width 0.3048) (layer F.Cu) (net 7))
 (segment (start 120.396 117.602) (end 122.428 119.634) (width 0.3048) (layer F.Cu) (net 7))
 (segment (start 120.396 114.3) (end 120.396 117.602) (width 0.3048) (layer F.Cu) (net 7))
 (segment (start 121.031 113.665) (end 120.396 114.3) (width 0.3048) (layer F.Cu) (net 7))
 (segment (start 123.444 121.92) (end 123.444 122.682) (width 0.3048) (layer F.Cu) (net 8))
 (segment (start 123.444 119.38) (end 121.412 117.348) (width 0.3048) (layer F.Cu) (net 8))
 (segment (start 122.428 114.935) (end 121.539 114.935) (width 0.3048) (layer F.Cu) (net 8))
 (segment (start 123.444 119.634) (end 123.444 121.92) (width 0.3048) (layer F.Cu) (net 8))
 (segment (start 121.158 117.094) (end 121.412 117.348) (width 0.3048) (layer F.Cu) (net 8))
 (segment (start 121.158 115.316) (end 121.158 117.094) (width 0.3048) (layer F.Cu) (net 8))
 (segment (start 121.539 114.935) (end 121.158 115.316) (width 0.3048) (layer F.Cu) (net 8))
 (segment (start 123.444 119.634) (end 123.444 119.38) (width 0.3048) (layer F.Cu) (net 8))
 (segment (start 125.476 124.714) (end 127.508 124.714) (width 0.3048) (layer F.Cu) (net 8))
 (segment (start 123.444 122.682) (end 125.476 124.714) (width 0.3048) (layer F.Cu) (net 8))
 (segment (start 120.396 111.76) (end 120.396 112.522) (width 0.3048) (layer F.Cu) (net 6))
 (segment (start 120.396 112.522) (end 119.888 113.03) (width 0.3048) (layer F.Cu) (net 6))
 (segment (start 119.888 113.03) (end 118.11 113.03) (width 0.3048) (layer F.Cu) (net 6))
 (segment (start 121.031 111.125) (end 120.396 111.76) (width 0.3048) (layer F.Cu) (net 6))
 (segment (start 122.428 111.125) (end 121.285 111.125) (width 0.3048) (layer F.Cu) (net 6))
 (segment (start 121.285 111.125) (end 121.031 111.125) (width 0.3048) (layer F.Cu) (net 6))
 (segment (start 120.396 108.458) (end 119.888 107.95) (width 0.3048) (layer F.Cu) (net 5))
 (segment (start 119.888 107.95) (end 118.11 107.95) (width 0.3048) (layer F.Cu) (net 5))
 (segment (start 121.031 109.855) (end 120.396 109.22) (width 0.3048) (layer F.Cu) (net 5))
 (segment (start 120.396 109.22) (end 120.396 108.458) (width 0.3048) (layer F.Cu) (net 5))
 (segment (start 122.428 109.855) (end 121.031 109.855) (width 0.3048) (layer F.Cu) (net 5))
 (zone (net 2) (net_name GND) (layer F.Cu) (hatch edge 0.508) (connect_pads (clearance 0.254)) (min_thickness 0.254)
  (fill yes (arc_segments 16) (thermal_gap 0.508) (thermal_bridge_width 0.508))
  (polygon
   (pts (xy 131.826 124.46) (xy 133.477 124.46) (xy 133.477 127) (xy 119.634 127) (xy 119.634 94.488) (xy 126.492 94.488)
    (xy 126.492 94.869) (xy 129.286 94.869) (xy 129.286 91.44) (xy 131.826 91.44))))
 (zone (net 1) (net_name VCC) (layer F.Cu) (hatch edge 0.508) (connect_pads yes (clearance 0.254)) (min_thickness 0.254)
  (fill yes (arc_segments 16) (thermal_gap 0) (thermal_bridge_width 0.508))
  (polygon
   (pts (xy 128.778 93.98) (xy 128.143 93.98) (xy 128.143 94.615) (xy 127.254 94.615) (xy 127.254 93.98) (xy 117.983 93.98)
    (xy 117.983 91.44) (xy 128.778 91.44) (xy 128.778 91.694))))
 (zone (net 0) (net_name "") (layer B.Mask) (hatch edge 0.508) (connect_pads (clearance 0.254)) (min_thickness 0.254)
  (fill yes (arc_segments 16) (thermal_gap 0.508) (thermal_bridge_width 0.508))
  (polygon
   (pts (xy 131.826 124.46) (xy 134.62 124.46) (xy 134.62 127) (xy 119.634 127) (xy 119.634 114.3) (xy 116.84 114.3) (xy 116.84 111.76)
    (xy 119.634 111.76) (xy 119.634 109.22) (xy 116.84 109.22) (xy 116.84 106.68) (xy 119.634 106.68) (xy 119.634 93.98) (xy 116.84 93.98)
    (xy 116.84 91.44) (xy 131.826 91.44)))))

